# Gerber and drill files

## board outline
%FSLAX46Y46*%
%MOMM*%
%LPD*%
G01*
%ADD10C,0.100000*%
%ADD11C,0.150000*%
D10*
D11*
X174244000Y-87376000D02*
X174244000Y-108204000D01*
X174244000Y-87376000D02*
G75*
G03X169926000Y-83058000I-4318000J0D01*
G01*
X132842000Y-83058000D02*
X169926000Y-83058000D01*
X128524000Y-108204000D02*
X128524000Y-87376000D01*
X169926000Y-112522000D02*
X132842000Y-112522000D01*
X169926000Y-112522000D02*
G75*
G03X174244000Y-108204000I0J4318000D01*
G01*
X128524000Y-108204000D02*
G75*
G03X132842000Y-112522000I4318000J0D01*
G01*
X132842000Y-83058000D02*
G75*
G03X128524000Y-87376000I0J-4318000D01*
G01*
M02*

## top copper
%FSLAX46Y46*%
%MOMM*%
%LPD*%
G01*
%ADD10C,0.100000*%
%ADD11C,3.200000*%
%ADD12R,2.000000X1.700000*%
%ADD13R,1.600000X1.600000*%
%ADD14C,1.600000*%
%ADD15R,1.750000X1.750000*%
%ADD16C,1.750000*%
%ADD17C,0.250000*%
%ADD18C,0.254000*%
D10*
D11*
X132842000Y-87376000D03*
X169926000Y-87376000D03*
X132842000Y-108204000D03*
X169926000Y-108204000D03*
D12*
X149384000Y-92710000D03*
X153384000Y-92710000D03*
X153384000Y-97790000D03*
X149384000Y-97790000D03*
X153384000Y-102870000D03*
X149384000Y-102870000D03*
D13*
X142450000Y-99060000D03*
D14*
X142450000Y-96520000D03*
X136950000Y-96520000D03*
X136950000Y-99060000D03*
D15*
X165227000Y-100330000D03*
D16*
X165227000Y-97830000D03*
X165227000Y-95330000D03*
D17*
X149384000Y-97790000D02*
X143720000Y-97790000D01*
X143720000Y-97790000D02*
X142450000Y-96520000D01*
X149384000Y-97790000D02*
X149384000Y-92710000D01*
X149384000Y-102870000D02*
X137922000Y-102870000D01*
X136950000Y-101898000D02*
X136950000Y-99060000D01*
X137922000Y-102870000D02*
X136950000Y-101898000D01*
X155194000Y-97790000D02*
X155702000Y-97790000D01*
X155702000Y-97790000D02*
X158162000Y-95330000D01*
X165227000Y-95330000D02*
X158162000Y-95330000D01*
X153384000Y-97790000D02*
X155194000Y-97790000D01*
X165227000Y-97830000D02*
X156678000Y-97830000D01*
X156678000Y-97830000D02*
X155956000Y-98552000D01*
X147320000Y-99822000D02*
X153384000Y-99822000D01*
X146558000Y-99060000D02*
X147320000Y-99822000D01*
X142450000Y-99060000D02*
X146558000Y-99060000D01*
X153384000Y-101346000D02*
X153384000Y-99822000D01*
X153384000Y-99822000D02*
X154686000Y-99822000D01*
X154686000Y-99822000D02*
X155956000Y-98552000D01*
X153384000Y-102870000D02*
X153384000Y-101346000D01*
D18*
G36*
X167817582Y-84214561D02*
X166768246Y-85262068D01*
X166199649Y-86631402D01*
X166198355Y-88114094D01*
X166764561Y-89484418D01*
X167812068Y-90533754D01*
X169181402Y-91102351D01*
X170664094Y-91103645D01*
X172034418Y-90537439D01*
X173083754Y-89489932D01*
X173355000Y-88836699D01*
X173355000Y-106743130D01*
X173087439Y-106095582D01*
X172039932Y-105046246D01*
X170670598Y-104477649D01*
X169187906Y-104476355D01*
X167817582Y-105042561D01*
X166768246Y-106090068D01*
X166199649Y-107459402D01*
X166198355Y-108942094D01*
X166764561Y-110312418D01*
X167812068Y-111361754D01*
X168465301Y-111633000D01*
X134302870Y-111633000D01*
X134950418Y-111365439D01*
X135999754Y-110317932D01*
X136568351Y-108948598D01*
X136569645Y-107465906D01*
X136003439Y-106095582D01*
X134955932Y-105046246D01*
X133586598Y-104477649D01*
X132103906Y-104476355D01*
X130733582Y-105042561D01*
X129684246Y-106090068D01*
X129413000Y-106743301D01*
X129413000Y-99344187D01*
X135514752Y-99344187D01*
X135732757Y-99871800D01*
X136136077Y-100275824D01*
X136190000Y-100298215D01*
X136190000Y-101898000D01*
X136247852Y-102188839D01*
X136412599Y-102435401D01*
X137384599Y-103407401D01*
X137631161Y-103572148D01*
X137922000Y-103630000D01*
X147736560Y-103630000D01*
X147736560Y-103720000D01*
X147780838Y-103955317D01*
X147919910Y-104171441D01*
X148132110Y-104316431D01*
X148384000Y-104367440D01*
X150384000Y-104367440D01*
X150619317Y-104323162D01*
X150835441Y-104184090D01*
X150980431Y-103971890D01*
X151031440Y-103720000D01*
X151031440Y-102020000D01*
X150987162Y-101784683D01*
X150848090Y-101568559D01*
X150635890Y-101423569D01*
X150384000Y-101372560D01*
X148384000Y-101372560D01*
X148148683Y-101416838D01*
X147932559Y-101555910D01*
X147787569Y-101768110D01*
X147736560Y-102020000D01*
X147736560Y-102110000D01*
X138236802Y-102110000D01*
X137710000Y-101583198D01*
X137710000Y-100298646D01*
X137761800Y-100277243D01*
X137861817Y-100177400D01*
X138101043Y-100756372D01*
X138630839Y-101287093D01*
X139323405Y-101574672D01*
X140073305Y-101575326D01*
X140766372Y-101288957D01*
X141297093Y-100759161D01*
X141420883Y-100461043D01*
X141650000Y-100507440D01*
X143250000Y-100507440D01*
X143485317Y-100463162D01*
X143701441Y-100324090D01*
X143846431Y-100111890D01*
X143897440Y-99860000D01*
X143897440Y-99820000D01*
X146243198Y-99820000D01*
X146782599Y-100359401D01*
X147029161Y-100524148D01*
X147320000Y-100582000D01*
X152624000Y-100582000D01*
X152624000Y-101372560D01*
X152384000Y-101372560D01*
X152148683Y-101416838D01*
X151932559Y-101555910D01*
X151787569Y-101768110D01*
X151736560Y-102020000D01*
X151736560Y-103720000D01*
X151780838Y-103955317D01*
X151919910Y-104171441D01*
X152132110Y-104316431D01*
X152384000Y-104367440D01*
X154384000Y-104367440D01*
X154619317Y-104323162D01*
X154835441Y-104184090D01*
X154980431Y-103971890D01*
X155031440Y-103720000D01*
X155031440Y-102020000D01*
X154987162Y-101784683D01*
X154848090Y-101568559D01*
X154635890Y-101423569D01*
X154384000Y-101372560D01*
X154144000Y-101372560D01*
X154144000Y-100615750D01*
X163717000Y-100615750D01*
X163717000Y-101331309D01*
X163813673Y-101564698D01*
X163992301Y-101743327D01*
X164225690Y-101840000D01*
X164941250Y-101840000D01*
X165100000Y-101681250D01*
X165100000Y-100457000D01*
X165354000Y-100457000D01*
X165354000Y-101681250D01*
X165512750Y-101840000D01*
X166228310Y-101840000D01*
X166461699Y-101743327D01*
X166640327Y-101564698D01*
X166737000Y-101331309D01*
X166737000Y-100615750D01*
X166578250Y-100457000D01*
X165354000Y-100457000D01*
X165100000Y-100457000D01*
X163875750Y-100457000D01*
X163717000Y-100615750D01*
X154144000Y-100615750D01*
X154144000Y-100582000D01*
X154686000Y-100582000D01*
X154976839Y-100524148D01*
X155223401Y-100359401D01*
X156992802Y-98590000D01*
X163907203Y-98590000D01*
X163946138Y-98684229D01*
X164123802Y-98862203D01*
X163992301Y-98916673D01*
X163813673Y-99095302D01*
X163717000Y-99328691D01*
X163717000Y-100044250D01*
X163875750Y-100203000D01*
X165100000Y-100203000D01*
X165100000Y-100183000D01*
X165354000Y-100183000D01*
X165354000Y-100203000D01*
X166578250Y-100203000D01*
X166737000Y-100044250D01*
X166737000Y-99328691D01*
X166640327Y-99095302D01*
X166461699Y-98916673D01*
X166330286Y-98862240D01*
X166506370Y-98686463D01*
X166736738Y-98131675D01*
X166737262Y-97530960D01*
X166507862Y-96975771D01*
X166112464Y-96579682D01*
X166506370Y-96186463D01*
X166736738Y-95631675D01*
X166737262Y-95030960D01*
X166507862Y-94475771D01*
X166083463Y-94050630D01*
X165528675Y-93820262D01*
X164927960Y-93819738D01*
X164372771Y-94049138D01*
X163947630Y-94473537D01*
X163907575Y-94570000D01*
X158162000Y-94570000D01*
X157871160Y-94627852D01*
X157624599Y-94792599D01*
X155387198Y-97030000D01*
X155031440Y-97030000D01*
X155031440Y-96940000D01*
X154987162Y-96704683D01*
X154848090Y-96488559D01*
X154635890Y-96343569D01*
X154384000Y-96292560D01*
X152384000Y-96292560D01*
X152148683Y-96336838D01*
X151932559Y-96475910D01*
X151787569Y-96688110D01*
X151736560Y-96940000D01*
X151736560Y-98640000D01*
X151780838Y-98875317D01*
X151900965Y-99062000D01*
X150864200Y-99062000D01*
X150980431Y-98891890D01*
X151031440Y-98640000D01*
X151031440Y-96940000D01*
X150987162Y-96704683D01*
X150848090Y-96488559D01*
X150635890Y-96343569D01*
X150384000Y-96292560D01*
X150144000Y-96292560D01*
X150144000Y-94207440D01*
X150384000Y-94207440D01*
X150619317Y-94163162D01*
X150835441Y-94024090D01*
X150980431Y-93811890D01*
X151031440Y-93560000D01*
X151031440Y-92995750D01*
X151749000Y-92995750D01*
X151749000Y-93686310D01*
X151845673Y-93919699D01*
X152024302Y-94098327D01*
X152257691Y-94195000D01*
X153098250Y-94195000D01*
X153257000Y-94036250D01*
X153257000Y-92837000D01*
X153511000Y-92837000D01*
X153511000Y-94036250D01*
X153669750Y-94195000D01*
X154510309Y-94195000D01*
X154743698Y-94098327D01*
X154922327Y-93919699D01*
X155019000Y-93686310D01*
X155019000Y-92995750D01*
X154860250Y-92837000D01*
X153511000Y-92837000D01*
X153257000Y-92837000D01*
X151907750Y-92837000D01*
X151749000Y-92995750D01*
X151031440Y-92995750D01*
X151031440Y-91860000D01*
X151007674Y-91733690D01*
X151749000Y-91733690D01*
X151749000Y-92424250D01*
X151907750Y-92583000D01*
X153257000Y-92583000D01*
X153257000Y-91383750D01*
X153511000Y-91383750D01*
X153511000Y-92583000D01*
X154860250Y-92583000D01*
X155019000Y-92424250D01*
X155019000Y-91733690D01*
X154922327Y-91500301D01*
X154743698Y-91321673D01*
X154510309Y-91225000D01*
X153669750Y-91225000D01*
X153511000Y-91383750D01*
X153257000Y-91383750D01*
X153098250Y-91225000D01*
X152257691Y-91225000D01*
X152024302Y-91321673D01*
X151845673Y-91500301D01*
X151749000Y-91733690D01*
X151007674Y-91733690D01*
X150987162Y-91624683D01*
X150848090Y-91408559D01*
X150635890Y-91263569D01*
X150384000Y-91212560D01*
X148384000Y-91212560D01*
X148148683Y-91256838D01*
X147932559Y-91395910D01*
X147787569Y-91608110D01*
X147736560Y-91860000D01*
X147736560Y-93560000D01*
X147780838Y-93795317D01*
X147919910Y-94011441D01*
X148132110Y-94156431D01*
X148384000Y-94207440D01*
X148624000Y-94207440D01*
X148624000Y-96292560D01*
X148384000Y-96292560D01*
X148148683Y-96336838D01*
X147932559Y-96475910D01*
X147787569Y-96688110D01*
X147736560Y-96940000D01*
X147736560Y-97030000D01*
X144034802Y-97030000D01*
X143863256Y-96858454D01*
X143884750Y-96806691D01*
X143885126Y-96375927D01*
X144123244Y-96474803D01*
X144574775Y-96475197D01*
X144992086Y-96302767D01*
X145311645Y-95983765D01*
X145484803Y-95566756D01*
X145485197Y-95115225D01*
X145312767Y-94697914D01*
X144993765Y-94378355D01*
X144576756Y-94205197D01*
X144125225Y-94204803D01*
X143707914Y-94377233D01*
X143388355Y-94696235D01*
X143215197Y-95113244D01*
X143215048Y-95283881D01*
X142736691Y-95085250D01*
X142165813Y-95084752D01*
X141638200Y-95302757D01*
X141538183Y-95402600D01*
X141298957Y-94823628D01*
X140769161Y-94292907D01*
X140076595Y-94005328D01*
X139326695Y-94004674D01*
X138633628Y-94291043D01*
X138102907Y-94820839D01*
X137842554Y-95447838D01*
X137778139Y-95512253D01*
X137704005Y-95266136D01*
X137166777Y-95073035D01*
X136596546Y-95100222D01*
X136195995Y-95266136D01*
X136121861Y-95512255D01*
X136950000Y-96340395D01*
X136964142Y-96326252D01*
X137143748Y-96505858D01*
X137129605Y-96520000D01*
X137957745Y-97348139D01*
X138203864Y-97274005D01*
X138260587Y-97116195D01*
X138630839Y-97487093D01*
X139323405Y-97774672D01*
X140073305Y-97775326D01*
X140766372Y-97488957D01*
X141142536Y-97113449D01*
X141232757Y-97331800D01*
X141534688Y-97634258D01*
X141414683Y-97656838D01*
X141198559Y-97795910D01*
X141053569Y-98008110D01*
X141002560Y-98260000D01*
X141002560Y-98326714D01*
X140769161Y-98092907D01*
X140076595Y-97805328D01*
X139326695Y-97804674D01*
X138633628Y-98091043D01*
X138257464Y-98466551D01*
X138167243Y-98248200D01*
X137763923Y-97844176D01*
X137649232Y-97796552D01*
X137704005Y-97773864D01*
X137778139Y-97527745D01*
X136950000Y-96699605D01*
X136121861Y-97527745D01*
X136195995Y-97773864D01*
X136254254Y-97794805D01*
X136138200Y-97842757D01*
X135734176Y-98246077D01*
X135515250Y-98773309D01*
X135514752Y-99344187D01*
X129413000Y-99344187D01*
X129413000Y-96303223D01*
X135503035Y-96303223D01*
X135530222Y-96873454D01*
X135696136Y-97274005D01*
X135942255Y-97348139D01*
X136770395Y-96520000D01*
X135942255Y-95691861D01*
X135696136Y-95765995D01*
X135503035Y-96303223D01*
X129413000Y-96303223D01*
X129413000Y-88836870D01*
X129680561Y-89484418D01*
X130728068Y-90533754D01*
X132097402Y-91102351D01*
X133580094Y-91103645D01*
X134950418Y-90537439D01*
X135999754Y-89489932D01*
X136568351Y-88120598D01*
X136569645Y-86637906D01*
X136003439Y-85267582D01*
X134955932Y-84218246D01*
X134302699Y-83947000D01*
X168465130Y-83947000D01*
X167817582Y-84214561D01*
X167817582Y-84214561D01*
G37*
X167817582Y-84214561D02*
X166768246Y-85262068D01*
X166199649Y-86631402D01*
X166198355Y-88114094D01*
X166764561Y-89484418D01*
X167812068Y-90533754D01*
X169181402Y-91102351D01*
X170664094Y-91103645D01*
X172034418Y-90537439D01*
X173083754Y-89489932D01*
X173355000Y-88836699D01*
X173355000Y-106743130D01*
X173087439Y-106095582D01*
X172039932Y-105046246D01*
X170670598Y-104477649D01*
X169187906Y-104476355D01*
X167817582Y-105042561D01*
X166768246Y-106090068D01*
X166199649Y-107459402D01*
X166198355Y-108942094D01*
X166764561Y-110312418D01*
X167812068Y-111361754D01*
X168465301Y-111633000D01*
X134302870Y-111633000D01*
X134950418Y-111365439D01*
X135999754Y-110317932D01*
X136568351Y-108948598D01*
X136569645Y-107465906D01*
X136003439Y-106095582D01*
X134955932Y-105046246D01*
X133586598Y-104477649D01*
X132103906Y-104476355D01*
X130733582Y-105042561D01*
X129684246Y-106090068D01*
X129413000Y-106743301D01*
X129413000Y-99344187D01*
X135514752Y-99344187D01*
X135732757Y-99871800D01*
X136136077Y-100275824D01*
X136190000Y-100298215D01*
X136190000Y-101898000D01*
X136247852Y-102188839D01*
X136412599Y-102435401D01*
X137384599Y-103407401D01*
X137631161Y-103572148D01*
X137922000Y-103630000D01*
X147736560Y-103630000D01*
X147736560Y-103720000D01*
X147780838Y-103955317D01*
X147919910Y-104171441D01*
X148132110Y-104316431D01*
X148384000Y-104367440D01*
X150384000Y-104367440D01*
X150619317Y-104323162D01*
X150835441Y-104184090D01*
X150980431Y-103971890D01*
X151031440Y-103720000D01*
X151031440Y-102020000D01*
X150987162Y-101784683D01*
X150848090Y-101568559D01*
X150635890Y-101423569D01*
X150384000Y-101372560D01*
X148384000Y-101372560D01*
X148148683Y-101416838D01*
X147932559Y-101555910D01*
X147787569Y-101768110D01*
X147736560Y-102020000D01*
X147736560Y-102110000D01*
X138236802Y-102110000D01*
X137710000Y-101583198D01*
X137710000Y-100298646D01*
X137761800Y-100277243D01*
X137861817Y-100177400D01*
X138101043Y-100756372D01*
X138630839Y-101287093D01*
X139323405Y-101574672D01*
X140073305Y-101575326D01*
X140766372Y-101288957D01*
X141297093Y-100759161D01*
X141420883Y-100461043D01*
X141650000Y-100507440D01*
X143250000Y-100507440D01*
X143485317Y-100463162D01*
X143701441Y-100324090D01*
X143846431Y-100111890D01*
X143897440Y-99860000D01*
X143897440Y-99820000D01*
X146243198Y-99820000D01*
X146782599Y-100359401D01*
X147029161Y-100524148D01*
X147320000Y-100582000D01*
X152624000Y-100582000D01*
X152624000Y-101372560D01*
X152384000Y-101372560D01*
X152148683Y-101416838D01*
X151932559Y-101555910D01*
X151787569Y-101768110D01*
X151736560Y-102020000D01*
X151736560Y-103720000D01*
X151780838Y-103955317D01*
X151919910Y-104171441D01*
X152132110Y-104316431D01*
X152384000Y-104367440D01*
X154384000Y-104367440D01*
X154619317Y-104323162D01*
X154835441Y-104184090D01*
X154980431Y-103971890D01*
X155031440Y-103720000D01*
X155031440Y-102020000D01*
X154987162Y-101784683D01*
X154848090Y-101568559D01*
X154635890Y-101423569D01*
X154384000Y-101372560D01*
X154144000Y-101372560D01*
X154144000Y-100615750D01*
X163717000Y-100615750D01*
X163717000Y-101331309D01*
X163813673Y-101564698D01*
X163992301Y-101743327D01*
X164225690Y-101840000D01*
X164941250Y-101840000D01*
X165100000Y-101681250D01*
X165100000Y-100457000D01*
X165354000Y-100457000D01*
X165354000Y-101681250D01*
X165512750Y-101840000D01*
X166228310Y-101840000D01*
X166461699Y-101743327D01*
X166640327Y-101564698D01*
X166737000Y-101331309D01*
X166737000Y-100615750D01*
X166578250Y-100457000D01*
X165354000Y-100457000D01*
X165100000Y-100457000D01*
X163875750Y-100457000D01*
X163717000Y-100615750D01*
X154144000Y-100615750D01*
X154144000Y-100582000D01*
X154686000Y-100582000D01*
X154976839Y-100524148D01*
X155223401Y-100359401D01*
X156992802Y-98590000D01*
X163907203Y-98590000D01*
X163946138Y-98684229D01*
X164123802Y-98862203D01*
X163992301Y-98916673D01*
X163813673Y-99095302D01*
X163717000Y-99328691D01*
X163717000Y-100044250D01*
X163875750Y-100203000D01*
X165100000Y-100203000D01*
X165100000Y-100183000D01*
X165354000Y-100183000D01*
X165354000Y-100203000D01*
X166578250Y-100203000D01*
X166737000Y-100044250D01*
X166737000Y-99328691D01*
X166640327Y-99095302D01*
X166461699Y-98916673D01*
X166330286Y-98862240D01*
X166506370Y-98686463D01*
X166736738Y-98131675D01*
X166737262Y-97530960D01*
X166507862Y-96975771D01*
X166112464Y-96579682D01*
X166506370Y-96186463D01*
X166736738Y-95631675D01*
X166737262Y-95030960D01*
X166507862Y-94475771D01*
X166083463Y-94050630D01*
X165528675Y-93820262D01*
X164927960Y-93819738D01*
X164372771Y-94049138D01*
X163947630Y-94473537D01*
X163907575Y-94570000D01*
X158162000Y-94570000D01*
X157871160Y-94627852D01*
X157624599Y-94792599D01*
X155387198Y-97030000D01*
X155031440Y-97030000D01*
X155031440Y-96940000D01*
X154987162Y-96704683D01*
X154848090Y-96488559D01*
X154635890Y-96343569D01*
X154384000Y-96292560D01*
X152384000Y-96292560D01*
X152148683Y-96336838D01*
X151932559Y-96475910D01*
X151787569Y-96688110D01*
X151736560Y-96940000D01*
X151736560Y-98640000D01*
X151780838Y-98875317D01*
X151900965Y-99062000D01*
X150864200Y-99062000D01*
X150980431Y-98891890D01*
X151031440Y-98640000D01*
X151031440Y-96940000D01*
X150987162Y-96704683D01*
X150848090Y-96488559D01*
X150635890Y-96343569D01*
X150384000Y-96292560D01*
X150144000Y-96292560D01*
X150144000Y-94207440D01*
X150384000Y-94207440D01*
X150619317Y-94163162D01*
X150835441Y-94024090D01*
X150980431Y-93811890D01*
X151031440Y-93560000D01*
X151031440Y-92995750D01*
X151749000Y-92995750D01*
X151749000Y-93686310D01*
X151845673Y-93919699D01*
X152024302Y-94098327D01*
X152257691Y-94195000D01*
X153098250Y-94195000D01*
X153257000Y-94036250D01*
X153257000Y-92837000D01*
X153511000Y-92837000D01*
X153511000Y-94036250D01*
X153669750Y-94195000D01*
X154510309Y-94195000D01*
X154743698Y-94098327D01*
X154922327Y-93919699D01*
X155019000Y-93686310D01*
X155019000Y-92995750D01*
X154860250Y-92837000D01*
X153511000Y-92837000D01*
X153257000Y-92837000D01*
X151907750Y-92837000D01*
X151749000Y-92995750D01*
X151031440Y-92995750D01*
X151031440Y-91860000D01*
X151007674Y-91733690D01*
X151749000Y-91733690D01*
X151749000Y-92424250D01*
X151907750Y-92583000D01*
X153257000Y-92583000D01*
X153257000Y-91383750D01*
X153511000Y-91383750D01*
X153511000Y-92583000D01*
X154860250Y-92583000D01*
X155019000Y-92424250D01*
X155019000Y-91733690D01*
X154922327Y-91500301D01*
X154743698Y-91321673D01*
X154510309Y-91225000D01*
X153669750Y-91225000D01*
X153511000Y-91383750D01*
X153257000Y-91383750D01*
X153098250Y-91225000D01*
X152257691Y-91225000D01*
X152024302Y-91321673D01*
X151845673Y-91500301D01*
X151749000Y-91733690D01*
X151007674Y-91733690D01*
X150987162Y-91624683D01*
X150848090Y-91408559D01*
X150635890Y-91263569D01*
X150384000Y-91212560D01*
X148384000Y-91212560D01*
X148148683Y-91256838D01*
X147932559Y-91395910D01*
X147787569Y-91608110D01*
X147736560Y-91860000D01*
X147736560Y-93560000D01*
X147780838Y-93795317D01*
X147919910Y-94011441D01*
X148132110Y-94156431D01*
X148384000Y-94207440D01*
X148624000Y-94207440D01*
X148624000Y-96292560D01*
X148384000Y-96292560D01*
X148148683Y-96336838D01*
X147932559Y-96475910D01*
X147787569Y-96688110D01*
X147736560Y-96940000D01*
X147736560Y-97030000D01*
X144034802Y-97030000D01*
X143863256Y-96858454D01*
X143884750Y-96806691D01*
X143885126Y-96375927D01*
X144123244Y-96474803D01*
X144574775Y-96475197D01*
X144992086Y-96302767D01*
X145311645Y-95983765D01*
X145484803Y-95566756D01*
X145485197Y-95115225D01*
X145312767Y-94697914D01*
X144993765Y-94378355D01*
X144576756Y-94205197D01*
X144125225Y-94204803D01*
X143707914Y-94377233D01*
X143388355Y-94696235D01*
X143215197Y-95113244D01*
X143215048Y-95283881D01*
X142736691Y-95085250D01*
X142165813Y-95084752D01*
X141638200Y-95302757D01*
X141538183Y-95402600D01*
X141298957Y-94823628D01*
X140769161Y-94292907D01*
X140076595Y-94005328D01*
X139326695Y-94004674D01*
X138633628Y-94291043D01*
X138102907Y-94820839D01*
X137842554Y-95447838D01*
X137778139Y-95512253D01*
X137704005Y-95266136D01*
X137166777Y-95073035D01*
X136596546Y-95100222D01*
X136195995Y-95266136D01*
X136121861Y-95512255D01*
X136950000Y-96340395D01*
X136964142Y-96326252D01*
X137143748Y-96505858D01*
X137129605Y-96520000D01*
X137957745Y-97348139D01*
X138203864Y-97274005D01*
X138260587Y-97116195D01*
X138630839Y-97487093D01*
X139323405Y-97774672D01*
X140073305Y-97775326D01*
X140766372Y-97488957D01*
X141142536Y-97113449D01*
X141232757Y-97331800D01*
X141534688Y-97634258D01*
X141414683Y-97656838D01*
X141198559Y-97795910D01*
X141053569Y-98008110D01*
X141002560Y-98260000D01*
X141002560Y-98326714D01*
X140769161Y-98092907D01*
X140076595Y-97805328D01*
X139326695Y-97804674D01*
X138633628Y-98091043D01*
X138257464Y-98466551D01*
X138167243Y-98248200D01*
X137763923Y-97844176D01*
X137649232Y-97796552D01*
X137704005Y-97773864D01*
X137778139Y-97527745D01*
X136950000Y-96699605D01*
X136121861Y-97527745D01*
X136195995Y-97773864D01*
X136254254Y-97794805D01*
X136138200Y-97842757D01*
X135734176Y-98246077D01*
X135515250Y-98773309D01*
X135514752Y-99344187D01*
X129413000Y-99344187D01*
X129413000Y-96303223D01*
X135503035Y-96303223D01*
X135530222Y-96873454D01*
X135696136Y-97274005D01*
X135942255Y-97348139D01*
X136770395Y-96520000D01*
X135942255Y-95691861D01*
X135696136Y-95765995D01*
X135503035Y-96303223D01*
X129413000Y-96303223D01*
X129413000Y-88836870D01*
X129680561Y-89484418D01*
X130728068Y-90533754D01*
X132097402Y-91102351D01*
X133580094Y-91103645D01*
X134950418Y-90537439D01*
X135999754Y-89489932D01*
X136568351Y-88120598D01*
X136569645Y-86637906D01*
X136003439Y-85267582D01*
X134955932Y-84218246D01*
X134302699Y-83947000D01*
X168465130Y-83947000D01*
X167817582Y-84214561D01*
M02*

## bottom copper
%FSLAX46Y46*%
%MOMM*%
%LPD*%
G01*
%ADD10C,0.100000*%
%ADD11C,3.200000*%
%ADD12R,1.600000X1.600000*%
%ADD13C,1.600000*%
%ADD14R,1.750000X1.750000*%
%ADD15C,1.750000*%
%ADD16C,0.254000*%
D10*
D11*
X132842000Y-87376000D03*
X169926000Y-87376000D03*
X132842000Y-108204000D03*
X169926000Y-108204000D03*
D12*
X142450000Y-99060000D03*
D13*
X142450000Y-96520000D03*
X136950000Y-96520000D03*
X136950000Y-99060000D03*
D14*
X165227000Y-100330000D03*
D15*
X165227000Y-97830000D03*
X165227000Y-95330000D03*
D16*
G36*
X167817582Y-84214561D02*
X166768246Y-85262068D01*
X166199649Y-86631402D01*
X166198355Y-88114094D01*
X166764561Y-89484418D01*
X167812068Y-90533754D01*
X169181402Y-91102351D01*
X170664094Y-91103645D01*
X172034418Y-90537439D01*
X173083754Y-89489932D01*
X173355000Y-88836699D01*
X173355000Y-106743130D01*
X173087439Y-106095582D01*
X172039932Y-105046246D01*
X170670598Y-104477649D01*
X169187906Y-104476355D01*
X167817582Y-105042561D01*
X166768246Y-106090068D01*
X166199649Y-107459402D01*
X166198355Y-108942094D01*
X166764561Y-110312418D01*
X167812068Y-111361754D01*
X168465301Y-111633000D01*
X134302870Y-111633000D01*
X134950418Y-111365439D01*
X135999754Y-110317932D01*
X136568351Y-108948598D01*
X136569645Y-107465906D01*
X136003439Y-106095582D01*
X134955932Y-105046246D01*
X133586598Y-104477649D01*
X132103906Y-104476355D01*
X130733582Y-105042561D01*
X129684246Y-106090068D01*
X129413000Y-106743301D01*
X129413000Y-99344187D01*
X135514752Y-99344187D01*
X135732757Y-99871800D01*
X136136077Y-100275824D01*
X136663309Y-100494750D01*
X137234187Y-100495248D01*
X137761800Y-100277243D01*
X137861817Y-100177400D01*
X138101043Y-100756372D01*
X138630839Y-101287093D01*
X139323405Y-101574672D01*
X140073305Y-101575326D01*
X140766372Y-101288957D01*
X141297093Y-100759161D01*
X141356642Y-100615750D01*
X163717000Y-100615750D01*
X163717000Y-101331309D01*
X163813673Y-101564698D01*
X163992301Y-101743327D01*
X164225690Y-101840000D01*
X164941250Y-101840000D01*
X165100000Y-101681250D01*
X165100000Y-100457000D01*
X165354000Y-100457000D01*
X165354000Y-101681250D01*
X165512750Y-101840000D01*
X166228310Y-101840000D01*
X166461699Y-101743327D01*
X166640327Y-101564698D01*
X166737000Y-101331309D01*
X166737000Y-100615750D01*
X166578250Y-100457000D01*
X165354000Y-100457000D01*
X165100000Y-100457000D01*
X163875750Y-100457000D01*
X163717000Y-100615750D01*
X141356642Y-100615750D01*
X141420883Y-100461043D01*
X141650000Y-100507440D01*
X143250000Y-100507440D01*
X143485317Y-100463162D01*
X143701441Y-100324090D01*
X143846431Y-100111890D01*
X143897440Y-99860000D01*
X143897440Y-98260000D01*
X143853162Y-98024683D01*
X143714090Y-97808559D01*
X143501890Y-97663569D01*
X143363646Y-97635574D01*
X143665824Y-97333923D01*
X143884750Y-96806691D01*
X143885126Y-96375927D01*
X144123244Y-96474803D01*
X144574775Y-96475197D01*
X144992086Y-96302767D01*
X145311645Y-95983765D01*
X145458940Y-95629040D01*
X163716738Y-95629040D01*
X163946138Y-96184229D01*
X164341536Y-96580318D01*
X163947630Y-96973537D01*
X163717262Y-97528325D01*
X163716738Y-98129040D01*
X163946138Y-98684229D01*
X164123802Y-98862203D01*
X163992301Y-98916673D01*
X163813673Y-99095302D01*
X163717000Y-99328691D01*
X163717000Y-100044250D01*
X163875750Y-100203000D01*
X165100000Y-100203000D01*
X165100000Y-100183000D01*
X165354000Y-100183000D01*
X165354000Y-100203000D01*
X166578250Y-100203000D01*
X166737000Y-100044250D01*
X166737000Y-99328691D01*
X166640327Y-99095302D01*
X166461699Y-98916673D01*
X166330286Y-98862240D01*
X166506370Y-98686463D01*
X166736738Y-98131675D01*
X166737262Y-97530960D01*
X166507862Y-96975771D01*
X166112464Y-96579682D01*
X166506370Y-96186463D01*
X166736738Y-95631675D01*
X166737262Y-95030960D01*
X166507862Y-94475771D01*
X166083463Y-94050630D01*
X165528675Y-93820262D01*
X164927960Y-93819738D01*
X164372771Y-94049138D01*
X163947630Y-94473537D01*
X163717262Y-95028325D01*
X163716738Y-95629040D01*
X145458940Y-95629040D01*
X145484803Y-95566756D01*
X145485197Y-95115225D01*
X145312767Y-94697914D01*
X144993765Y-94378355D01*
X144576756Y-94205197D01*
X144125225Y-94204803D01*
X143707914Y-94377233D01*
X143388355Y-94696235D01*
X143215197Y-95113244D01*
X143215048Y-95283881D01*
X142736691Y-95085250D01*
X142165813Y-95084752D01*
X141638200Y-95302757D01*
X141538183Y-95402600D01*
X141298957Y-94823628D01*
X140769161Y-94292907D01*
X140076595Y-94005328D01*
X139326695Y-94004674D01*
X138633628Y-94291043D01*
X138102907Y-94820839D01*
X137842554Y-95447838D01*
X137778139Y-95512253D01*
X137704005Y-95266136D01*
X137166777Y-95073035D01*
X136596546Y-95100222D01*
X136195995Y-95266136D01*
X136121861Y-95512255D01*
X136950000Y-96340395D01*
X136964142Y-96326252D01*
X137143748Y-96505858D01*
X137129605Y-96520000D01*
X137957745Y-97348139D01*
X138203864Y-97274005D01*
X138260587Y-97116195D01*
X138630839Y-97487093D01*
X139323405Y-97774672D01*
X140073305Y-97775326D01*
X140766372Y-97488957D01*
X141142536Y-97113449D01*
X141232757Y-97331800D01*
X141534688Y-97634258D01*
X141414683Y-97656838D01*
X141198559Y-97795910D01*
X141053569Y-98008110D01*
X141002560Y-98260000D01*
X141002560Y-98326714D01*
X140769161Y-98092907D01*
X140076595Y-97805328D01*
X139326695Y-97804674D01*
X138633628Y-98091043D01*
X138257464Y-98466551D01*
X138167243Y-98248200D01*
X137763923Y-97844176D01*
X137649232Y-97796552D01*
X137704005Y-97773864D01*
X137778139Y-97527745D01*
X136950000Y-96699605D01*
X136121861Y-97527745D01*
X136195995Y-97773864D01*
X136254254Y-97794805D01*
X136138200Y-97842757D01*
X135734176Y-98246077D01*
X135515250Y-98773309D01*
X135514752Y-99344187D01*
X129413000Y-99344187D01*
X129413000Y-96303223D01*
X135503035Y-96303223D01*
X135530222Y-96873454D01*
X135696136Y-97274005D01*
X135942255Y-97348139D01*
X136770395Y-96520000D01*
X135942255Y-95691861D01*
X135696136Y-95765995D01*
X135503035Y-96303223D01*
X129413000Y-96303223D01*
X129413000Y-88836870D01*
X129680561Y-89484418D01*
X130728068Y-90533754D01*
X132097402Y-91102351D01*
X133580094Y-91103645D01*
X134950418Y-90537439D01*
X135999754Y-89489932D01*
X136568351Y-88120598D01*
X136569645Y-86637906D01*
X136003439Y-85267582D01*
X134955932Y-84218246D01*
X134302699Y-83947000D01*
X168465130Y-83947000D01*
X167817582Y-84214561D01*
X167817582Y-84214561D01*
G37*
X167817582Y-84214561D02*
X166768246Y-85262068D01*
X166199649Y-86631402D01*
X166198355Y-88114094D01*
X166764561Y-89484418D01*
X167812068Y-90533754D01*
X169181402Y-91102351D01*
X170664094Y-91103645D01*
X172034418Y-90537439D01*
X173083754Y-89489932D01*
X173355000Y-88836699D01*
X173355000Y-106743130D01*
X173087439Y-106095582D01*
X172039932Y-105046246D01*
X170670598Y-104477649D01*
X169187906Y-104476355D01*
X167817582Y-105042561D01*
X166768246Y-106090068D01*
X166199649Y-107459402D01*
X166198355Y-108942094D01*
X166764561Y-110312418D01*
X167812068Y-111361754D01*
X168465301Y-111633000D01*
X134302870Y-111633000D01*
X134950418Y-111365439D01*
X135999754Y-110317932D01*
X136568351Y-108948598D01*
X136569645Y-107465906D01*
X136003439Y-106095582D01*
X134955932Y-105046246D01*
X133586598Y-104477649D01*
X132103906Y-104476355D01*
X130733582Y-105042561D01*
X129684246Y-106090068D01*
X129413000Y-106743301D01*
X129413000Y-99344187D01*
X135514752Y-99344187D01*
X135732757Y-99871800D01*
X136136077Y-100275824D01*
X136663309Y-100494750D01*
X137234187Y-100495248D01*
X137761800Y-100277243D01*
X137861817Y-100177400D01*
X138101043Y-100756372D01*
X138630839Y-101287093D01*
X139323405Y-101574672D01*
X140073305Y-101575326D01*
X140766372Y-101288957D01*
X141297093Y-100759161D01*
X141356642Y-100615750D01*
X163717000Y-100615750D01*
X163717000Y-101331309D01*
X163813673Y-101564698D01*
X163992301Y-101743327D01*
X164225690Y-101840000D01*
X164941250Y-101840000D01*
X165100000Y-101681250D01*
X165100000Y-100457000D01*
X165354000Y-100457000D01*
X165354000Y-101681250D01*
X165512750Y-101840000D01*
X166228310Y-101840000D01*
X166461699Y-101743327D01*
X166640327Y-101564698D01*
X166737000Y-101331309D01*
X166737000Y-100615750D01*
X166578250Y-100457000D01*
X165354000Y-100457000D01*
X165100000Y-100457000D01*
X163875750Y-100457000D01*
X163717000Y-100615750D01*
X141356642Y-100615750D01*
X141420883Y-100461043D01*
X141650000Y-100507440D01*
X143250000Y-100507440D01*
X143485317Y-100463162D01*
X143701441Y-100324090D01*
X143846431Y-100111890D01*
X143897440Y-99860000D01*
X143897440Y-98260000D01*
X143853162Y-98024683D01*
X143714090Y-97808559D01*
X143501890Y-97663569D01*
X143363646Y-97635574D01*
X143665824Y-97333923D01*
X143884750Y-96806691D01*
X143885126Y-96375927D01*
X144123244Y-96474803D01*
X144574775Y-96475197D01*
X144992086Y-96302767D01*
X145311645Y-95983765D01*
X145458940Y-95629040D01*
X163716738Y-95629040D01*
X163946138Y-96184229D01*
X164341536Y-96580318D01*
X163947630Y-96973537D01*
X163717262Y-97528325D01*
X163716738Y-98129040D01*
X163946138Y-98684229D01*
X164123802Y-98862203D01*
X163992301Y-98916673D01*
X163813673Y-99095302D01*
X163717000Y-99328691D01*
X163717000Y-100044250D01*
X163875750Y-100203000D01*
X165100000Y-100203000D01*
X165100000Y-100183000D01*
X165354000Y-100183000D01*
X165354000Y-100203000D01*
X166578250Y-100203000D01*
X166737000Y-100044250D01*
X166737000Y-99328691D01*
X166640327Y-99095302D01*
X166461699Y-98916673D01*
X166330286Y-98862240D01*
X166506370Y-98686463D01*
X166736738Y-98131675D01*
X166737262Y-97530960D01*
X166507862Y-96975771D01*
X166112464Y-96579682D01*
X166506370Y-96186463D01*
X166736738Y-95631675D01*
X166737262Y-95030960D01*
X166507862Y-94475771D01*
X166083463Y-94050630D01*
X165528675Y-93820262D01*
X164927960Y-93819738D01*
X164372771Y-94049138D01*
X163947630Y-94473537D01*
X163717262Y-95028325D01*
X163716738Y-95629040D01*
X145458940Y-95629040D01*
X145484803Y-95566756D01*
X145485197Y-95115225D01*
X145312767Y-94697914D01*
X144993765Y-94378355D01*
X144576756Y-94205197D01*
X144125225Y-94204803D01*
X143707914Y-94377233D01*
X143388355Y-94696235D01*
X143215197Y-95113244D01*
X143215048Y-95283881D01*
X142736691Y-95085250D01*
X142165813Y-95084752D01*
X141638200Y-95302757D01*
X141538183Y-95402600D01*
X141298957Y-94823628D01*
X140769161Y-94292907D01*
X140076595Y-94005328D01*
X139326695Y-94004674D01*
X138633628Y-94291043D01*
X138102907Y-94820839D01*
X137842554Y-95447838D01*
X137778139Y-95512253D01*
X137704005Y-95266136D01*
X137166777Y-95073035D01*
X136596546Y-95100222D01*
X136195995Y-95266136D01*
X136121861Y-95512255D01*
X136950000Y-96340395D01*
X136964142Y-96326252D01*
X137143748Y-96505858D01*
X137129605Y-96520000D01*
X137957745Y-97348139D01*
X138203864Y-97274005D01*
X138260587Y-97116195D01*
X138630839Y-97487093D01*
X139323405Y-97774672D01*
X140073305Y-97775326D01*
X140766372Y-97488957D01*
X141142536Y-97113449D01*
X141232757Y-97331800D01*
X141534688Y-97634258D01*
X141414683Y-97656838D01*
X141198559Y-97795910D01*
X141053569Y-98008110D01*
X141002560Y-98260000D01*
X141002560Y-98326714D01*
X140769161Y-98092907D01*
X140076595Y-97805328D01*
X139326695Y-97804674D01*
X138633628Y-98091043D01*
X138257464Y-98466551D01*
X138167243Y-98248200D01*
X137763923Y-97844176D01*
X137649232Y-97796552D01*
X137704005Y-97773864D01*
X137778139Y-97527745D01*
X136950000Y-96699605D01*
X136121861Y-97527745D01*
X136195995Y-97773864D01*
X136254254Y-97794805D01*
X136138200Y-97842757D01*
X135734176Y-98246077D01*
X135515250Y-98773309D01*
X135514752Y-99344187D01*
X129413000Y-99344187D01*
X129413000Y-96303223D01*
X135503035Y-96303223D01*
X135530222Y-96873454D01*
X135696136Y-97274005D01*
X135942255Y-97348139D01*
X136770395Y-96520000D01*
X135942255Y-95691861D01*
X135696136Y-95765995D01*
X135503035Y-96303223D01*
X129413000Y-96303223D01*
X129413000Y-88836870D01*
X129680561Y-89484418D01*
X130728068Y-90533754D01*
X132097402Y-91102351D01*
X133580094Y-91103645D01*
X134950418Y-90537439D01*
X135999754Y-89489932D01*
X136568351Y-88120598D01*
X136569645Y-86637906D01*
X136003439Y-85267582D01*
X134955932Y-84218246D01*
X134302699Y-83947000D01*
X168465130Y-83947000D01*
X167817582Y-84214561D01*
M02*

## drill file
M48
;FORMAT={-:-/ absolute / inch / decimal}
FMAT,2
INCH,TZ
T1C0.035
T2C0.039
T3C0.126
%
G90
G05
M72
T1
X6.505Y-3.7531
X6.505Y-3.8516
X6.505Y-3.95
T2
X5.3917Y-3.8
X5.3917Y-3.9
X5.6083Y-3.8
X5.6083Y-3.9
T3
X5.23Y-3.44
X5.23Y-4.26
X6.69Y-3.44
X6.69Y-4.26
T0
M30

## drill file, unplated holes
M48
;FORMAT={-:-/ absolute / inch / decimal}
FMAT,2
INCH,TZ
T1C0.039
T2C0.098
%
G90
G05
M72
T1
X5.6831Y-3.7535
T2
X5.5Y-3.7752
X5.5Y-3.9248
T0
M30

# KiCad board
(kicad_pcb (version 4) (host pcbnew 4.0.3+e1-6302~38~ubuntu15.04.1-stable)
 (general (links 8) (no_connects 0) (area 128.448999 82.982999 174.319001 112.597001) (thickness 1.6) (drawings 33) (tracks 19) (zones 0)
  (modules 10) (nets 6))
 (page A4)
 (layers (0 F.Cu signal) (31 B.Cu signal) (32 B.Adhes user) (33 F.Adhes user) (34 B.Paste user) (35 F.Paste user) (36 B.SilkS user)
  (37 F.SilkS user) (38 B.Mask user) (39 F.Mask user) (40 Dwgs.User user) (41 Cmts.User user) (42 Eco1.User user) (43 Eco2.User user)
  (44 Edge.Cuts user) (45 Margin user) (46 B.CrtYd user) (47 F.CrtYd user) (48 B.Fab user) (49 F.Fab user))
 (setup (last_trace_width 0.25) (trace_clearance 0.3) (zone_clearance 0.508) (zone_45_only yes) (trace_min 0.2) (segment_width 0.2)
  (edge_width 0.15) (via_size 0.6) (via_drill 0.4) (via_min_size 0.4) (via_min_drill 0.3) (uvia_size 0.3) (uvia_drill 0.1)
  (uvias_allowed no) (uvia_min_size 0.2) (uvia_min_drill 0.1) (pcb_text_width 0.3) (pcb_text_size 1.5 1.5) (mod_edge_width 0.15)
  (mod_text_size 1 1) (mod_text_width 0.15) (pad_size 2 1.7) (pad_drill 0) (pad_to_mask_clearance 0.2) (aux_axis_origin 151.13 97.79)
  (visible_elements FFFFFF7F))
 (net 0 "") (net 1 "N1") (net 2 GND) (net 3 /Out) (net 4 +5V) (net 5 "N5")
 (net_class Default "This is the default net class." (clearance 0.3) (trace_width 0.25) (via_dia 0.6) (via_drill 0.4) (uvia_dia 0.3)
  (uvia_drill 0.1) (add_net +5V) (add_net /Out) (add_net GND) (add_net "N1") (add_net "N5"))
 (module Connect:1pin (layer F.Cu) (at 132.842 87.376)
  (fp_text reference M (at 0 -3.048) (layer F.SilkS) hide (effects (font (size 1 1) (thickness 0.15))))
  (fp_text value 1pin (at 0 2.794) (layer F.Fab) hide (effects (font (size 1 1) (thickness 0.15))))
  (pad 1 thru_hole circle (at 0 0) (size 3.2 3.2) (drill 3.2) (layers *.Cu *.Mask F.SilkS) (clearance 2)))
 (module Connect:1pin (layer F.Cu) (at 169.926 87.376)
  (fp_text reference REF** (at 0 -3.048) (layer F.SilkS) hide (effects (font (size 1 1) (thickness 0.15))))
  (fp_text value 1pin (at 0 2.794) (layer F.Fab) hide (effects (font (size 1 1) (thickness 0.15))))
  (pad 1 thru_hole circle (at 0 0) (size 3.2 3.2) (drill 3.2) (layers *.Cu *.Mask F.SilkS) (clearance 2)))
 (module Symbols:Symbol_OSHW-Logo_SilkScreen (layer B.Cu) (at 151.384 97.028 180)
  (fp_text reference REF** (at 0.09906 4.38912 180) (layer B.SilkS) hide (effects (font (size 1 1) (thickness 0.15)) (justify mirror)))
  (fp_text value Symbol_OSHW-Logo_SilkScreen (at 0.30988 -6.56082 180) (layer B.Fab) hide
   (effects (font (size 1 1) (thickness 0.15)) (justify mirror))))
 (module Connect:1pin (layer F.Cu) (at 132.842 108.204)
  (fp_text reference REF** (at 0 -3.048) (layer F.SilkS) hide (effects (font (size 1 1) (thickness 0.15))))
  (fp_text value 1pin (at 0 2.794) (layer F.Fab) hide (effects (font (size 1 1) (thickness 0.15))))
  (pad 1 thru_hole circle (at 0 0) (size 3.2 3.2) (drill 3.2) (layers *.Cu *.Mask F.SilkS) (clearance 2)))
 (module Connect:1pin (layer F.Cu) (at 169.926 108.204)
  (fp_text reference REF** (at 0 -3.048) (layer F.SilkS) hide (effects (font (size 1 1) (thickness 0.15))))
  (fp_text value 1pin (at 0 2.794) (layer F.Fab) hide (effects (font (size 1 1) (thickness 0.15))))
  (pad 1 thru_hole circle (at 0 0) (size 3.2 3.2) (drill 3.2) (layers *.Cu *.Mask F.SilkS) (clearance 2)))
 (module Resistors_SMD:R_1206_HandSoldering (layer F.Cu) (at 151.384 92.71)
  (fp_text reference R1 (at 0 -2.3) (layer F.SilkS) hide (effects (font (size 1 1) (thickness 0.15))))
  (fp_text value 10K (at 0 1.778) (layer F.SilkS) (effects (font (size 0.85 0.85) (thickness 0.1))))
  (pad 1 smd rect (at -2 0) (size 2 1.7) (layers F.Cu F.Paste F.Mask) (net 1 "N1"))
  (pad 2 smd rect (at 2 0) (size 2 1.7) (layers F.Cu F.Paste F.Mask) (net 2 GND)))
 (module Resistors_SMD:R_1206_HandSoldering (layer F.Cu) (at 151.384 97.79 180)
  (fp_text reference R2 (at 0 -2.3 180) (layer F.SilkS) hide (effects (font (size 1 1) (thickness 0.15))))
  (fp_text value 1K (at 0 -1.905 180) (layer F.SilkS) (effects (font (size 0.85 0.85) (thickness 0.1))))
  (pad 1 smd rect (at -2 0 180) (size 2 1.7) (layers F.Cu F.Paste F.Mask) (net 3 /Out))
  (pad 2 smd rect (at 2 0 180) (size 2 1.7) (layers F.Cu F.Paste F.Mask) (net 1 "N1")))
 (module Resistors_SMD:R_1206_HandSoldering (layer F.Cu) (at 151.384 102.87 180)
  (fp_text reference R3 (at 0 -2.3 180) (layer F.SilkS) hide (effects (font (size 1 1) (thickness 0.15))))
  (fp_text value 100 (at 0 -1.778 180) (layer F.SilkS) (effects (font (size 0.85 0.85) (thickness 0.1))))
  (pad 1 smd rect (at -2 0 180) (size 2 1.7) (layers F.Cu F.Paste F.Mask) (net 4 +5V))
  (pad 2 smd rect (at 2 0 180) (size 2 1.7) (layers F.Cu F.Paste F.Mask) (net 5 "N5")))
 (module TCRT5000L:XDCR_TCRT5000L (layer F.Cu) (at 139.7 97.79 180) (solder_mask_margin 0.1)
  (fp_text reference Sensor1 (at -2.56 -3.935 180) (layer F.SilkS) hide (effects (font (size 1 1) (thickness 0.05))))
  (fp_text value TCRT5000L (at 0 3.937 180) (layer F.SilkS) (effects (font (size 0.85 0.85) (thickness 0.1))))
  (pad 1 thru_hole rect (at -2.75 -1.27 180) (size 1.6 1.6) (drill 1) (layers *.Cu *.Mask F.SilkS) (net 4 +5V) (solder_mask_margin 0.2))
  (pad 2 thru_hole circle (at -2.75 1.27 180) (size 1.6 1.6) (drill 1) (layers *.Cu *.Mask F.SilkS) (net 1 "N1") (solder_mask_margin 0.2))
  (pad 3 thru_hole circle (at 2.75 1.27 180) (size 1.6 1.6) (drill 1) (layers *.Cu *.Mask F.SilkS) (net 2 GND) (solder_mask_margin 0.2))
  (pad 4 thru_hole circle (at 2.75 -1.27 180) (size 1.6 1.6) (drill 1) (layers *.Cu *.Mask F.SilkS) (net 5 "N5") (solder_mask_margin 0.2))
  (pad Hole np_thru_hole circle (at 0 -1.9 180) (size 2.5 2.5) (drill 2.5) (layers))
  (pad Hole np_thru_hole circle (at 0 1.9 180) (size 2.5 2.5) (drill 2.5) (layers))
  (pad Hole np_thru_hole circle (at -4.65 2.45 180) (size 1 1) (drill 1) (layers)))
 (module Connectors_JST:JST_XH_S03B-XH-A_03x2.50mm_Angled (layer F.Cu) (at 165.227 100.33 90)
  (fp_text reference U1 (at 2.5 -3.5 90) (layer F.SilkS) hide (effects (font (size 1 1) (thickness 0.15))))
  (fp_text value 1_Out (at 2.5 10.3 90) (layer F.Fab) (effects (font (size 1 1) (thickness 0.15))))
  (pad 1 thru_hole rect (at 0 0 90) (size 1.75 1.75) (drill 0.9) (layers *.Cu *.Mask F.SilkS) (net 2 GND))
  (pad 2 thru_hole circle (at 2.5 0 90) (size 1.75 1.75) (drill 0.9) (layers *.Cu *.Mask F.SilkS) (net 4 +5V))
  (pad 3 thru_hole circle (at 5 0 90) (size 1.75 1.75) (drill 0.9) (layers *.Cu *.Mask F.SilkS) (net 3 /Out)))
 (gr_line (start 174.244 87.376) (end 174.244 108.204) (angle 90) (layer Edge.Cuts) (width 0.15))
 (gr_arc (start 169.926 87.376) (end 169.926 83.058) (angle 90) (layer Edge.Cuts) (width 0.15))
 (gr_line (start 132.842 83.058) (end 169.926 83.058) (angle 90) (layer Edge.Cuts) (width 0.15))
 (gr_line (start 128.524 108.204) (end 128.524 87.376) (angle 90) (layer Edge.Cuts) (width 0.15))
 (gr_line (start 169.926 112.522) (end 132.842 112.522) (angle 90) (layer Edge.Cuts) (width 0.15))
 (gr_arc (start 169.926 108.204) (end 174.244 108.204) (angle 90) (layer Edge.Cuts) (width 0.15))
 (gr_arc (start 132.842 108.204) (end 132.842 112.522) (angle 90) (layer Edge.Cuts) (width 0.15))
 (gr_arc (start 132.842 87.376) (end 128.524 87.376) (angle 90) (layer Edge.Cuts) (width 0.15))
 (segment (start 149.384 97.79) (end 143.72 97.79) (width 0.25) (layer F.Cu) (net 1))
 (segment (start 143.72 97.79) (end 142.45 96.52) (width 0.25) (layer F.Cu) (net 1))
 (segment (start 149.384 97.79) (end 149.384 92.71) (width 0.25) (layer F.Cu) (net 1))
 (segment (start 149.384 102.87) (end 137.922 102.87) (width 0.25) (layer F.Cu) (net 5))
 (segment (start 136.95 101.898) (end 136.95 99.06) (width 0.25) (layer F.Cu) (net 5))
 (segment (start 137.922 102.87) (end 136.95 101.898) (width 0.25) (layer F.Cu) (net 5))
 (segment (start 155.194 97.79) (end 155.702 97.79) (width 0.25) (layer F.Cu) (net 3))
 (segment (start 155.702 97.79) (end 158.162 95.33) (width 0.25) (layer F.Cu) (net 3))
 (segment (start 165.227 95.33) (end 158.162 95.33) (width 0.25) (layer F.Cu) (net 3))
 (segment (start 153.384 97.79) (end 155.194 97.79) (width 0.25) (layer F.Cu) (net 3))
 (segment (start 165.227 97.83) (end 156.678 97.83) (width 0.25) (layer F.Cu) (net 4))
 (segment (start 156.678 97.83) (end 155.956 98.552) (width 0.25) (layer F.Cu) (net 4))
 (segment (start 147.32 99.822) (end 153.384 99.822) (width 0.25) (layer F.Cu) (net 4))
 (segment (start 146.558 99.06) (end 147.32 99.822) (width 0.25) (layer F.Cu) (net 4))
 (segment (start 142.45 99.06) (end 146.558 99.06) (width 0.25) (layer F.Cu) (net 4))
 (segment (start 153.384 101.346) (end 153.384 99.822) (width 0.25) (layer F.Cu) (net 4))
 (segment (start 153.384 99.822) (end 154.686 99.822) (width 0.25) (layer F.Cu) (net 4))
 (segment (start 154.686 99.822) (end 155.956 98.552) (width 0.25) (layer F.Cu) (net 4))
 (segment (start 153.384 102.87) (end 153.384 101.346) (width 0.25) (layer F.Cu) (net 4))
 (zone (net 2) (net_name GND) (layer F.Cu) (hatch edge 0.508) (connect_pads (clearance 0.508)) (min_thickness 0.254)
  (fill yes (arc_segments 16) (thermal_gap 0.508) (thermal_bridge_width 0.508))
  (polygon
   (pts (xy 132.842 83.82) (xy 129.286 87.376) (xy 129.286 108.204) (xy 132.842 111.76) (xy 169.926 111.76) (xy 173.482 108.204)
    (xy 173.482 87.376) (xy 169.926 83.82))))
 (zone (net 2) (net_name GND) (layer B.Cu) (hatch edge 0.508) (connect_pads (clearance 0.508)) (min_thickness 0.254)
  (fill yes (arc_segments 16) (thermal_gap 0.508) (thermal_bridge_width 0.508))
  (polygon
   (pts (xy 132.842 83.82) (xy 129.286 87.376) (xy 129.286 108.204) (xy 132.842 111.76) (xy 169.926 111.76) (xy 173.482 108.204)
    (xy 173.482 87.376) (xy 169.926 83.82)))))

